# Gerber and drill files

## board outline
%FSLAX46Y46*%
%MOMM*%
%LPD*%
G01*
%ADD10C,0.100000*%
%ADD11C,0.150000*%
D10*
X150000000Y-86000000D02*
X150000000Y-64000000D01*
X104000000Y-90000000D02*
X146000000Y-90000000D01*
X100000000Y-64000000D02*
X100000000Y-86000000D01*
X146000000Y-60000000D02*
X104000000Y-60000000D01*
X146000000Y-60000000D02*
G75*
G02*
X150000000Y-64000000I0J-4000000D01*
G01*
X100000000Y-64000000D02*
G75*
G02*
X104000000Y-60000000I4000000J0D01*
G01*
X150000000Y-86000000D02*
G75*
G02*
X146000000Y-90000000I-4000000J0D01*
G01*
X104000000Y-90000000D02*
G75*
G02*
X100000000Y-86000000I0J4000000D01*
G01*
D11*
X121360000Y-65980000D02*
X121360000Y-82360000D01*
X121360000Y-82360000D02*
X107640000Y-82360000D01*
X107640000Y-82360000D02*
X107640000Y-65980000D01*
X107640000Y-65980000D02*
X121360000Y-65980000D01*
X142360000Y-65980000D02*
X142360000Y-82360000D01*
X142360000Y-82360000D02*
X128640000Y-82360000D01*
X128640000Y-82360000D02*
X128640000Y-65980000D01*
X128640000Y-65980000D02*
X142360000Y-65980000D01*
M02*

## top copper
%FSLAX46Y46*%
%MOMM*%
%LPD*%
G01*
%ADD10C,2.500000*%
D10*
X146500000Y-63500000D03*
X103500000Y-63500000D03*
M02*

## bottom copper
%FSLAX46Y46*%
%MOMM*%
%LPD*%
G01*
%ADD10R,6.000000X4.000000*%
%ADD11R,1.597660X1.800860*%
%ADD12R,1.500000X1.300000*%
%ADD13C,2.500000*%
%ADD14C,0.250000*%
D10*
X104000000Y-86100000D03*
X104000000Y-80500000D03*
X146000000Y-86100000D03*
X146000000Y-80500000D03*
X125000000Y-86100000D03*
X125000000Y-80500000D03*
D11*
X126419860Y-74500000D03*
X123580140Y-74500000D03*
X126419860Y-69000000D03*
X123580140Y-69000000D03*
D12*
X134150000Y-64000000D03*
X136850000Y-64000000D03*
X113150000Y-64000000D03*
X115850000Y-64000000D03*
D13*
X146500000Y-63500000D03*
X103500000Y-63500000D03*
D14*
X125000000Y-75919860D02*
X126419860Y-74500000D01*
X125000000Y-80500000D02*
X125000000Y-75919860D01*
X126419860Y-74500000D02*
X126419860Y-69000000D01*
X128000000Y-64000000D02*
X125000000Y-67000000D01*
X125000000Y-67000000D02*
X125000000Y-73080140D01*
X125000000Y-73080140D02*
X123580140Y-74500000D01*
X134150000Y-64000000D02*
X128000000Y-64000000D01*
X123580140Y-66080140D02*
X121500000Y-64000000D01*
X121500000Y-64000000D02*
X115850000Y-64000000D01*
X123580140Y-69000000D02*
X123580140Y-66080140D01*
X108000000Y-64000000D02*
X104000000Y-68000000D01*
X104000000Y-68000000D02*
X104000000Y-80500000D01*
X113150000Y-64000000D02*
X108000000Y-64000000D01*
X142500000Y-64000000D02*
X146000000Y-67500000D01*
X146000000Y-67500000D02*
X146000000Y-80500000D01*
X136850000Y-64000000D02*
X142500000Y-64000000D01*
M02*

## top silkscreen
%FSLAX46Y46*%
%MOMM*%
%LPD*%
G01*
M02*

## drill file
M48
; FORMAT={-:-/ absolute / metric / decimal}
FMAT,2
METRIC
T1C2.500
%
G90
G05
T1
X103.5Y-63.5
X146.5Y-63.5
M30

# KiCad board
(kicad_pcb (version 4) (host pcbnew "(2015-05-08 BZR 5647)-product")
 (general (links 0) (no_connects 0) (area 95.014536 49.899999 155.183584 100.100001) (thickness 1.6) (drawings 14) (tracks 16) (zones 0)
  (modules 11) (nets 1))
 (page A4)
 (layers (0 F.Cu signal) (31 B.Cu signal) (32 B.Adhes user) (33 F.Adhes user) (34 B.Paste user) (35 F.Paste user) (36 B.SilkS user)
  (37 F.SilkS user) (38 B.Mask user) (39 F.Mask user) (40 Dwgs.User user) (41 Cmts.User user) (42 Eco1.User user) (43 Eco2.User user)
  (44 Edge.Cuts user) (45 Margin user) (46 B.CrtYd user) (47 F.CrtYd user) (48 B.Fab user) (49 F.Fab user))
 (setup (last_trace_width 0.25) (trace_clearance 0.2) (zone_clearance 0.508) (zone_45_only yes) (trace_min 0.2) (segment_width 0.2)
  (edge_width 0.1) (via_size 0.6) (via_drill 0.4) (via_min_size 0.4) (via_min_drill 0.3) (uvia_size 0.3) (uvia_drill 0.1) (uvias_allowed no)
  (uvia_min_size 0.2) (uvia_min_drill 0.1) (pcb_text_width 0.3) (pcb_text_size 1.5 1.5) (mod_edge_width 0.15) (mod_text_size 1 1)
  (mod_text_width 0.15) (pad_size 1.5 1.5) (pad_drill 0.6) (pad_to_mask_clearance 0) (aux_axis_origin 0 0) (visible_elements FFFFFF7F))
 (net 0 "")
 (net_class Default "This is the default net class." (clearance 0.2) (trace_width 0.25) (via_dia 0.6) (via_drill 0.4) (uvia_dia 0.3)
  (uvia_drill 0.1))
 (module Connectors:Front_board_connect (layer F.Cu) (at 104 82.5)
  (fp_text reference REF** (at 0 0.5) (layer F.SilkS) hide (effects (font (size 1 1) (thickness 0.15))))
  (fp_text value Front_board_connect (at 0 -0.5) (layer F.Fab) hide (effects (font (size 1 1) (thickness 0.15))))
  (pad 1 smd rect (at 0 3.6) (size 6 4) (layers B.Cu B.Paste B.Mask))
  (pad 2 smd rect (at 0 -2) (size 6 4) (layers B.Cu B.Paste B.Mask)))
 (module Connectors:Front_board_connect (layer F.Cu) (at 146 82.5)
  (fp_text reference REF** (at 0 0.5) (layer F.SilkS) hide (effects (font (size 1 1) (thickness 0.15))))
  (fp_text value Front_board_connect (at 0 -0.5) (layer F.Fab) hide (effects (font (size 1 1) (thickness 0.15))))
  (pad 1 smd rect (at 0 3.6) (size 6 4) (layers B.Cu B.Paste B.Mask))
  (pad 2 smd rect (at 0 -2) (size 6 4) (layers B.Cu B.Paste B.Mask)))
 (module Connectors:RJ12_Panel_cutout (layer F.Cu) (at 114.5 83)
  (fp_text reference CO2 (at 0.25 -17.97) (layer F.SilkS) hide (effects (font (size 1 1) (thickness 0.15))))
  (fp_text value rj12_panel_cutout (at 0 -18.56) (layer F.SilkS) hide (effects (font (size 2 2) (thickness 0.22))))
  (fp_line (start 6.86 -17.02) (end 6.86 -0.64) (layer Edge.Cuts) (width 0.15))
  (fp_line (start 6.86 -0.64) (end -6.86 -0.64) (layer Edge.Cuts) (width 0.15))
  (fp_line (start -6.86 -0.64) (end -6.86 -17.02) (layer Edge.Cuts) (width 0.15))
  (fp_line (start -6.86 -17.02) (end 6.86 -17.02) (layer Edge.Cuts) (width 0.15)))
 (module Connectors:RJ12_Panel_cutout (layer F.Cu) (at 135.5 83)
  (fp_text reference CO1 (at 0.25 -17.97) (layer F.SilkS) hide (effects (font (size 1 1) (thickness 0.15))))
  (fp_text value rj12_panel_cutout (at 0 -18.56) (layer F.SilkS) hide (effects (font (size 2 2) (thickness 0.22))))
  (fp_line (start 6.86 -17.02) (end 6.86 -0.64) (layer Edge.Cuts) (width 0.15))
  (fp_line (start 6.86 -0.64) (end -6.86 -0.64) (layer Edge.Cuts) (width 0.15))
  (fp_line (start -6.86 -0.64) (end -6.86 -17.02) (layer Edge.Cuts) (width 0.15))
  (fp_line (start -6.86 -17.02) (end 6.86 -17.02) (layer Edge.Cuts) (width 0.15)))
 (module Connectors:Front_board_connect (layer F.Cu) (at 125 82.5)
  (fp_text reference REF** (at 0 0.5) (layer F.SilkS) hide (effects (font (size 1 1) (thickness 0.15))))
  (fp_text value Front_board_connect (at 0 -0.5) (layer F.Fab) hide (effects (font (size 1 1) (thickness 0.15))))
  (pad 1 smd rect (at 0 3.6) (size 6 4) (layers B.Cu B.Paste B.Mask))
  (pad 2 smd rect (at 0 -2) (size 6 4) (layers B.Cu B.Paste B.Mask)))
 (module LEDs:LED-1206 (layer B.Cu) (at 125 74.5)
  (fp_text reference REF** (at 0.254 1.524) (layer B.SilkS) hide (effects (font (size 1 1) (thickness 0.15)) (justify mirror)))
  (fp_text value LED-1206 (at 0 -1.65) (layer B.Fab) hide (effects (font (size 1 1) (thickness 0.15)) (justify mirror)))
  (pad 2 smd rect (at 1.41986 0 180) (size 1.59766 1.80086) (layers B.Cu B.Paste B.Mask))
  (pad 1 smd rect (at -1.41986 0 180) (size 1.59766 1.80086) (layers B.Cu B.Paste B.Mask)))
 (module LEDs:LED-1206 (layer B.Cu) (at 125 69)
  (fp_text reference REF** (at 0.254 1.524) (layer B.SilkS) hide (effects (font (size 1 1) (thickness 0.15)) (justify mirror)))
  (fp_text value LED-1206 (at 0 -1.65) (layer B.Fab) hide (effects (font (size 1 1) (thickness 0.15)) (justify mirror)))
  (pad 2 smd rect (at 1.41986 0 180) (size 1.59766 1.80086) (layers B.Cu B.Paste B.Mask))
  (pad 1 smd rect (at -1.41986 0 180) (size 1.59766 1.80086) (layers B.Cu B.Paste B.Mask)))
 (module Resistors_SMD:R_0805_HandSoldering (layer B.Cu) (at 135.5 64)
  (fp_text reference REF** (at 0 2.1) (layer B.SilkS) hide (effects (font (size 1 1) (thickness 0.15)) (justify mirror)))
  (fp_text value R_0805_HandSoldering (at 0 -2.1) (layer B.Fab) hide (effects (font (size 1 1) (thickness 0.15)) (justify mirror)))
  (pad 1 smd rect (at -1.35 0) (size 1.5 1.3) (layers B.Cu B.Paste B.Mask))
  (pad 2 smd rect (at 1.35 0) (size 1.5 1.3) (layers B.Cu B.Paste B.Mask)))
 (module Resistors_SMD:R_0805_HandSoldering (layer B.Cu) (at 114.5 64)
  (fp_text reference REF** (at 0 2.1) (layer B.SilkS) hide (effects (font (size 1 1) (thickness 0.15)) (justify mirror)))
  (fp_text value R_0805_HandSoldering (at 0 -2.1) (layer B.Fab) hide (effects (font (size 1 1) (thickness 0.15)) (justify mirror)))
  (pad 1 smd rect (at -1.35 0) (size 1.5 1.3) (layers B.Cu B.Paste B.Mask))
  (pad 2 smd rect (at 1.35 0) (size 1.5 1.3) (layers B.Cu B.Paste B.Mask)))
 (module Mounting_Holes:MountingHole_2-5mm (layer F.Cu) (at 146.5 63.5)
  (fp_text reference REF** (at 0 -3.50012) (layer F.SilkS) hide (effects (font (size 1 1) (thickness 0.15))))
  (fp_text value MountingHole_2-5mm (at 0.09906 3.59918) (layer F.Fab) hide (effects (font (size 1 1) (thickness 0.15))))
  (pad 1 thru_hole circle (at 0 0) (size 2.5 2.5) (drill 2.5) (layers)))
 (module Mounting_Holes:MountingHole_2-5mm (layer F.Cu) (at 103.5 63.5)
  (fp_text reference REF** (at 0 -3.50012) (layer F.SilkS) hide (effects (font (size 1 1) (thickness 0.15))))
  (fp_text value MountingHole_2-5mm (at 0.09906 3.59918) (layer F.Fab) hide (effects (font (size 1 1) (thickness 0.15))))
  (pad 1 thru_hole circle (at 0 0) (size 2.5 2.5) (drill 2.5) (layers)))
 (gr_line (start 150 86) (end 150 64) (angle 90) (layer Edge.Cuts) (width 0.1))
 (gr_line (start 104 90) (end 146 90) (angle 90) (layer Edge.Cuts) (width 0.1))
 (gr_line (start 100 64) (end 100 86) (angle 90) (layer Edge.Cuts) (width 0.1))
 (gr_line (start 146 60) (end 104 60) (angle 90) (layer Edge.Cuts) (width 0.1))
 (gr_arc (start 146 64) (end 146 60) (angle 90) (layer Edge.Cuts) (width 0.1))
 (gr_arc (start 104 64) (end 100 64) (angle 90) (layer Edge.Cuts) (width 0.1))
 (gr_arc (start 146 86) (end 150 86) (angle 90) (layer Edge.Cuts) (width 0.1))
 (gr_arc (start 104 86) (end 104 90) (angle 90) (layer Edge.Cuts) (width 0.1))
 (segment (start 125 75.91986) (end 126.41986 74.5) (width 0.25) (layer B.Cu) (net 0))
 (segment (start 125 80.5) (end 125 75.91986) (width 0.25) (layer B.Cu) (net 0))
 (segment (start 126.41986 74.5) (end 126.41986 69) (width 0.25) (layer B.Cu) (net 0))
 (segment (start 128 64) (end 125 67) (width 0.25) (layer B.Cu) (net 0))
 (segment (start 125 67) (end 125 73.08014) (width 0.25) (layer B.Cu) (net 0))
 (segment (start 125 73.08014) (end 123.58014 74.5) (width 0.25) (layer B.Cu) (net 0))
 (segment (start 134.15 64) (end 128 64) (width 0.25) (layer B.Cu) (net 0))
 (segment (start 123.58014 66.08014) (end 121.5 64) (width 0.25) (layer B.Cu) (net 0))
 (segment (start 121.5 64) (end 115.85 64) (width 0.25) (layer B.Cu) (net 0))
 (segment (start 123.58014 69) (end 123.58014 66.08014) (width 0.25) (layer B.Cu) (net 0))
 (segment (start 108 64) (end 104 68) (width 0.25) (layer B.Cu) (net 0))
 (segment (start 104 68) (end 104 80.5) (width 0.25) (layer B.Cu) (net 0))
 (segment (start 113.15 64) (end 108 64) (width 0.25) (layer B.Cu) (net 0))
 (segment (start 142.5 64) (end 146 67.5) (width 0.25) (layer B.Cu) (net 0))
 (segment (start 146 67.5) (end 146 80.5) (width 0.25) (layer B.Cu) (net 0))
 (segment (start 136.85 64) (end 142.5 64) (width 0.25) (layer B.Cu) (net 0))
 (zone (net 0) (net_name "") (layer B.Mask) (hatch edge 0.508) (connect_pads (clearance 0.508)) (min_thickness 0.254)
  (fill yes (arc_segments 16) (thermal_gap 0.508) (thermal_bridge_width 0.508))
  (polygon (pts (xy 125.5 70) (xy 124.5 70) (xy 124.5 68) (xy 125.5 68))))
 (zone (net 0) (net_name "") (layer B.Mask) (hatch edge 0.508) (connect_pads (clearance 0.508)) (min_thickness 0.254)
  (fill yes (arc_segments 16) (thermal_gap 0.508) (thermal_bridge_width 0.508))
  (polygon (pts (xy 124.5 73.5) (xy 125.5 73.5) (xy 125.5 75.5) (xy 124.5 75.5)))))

